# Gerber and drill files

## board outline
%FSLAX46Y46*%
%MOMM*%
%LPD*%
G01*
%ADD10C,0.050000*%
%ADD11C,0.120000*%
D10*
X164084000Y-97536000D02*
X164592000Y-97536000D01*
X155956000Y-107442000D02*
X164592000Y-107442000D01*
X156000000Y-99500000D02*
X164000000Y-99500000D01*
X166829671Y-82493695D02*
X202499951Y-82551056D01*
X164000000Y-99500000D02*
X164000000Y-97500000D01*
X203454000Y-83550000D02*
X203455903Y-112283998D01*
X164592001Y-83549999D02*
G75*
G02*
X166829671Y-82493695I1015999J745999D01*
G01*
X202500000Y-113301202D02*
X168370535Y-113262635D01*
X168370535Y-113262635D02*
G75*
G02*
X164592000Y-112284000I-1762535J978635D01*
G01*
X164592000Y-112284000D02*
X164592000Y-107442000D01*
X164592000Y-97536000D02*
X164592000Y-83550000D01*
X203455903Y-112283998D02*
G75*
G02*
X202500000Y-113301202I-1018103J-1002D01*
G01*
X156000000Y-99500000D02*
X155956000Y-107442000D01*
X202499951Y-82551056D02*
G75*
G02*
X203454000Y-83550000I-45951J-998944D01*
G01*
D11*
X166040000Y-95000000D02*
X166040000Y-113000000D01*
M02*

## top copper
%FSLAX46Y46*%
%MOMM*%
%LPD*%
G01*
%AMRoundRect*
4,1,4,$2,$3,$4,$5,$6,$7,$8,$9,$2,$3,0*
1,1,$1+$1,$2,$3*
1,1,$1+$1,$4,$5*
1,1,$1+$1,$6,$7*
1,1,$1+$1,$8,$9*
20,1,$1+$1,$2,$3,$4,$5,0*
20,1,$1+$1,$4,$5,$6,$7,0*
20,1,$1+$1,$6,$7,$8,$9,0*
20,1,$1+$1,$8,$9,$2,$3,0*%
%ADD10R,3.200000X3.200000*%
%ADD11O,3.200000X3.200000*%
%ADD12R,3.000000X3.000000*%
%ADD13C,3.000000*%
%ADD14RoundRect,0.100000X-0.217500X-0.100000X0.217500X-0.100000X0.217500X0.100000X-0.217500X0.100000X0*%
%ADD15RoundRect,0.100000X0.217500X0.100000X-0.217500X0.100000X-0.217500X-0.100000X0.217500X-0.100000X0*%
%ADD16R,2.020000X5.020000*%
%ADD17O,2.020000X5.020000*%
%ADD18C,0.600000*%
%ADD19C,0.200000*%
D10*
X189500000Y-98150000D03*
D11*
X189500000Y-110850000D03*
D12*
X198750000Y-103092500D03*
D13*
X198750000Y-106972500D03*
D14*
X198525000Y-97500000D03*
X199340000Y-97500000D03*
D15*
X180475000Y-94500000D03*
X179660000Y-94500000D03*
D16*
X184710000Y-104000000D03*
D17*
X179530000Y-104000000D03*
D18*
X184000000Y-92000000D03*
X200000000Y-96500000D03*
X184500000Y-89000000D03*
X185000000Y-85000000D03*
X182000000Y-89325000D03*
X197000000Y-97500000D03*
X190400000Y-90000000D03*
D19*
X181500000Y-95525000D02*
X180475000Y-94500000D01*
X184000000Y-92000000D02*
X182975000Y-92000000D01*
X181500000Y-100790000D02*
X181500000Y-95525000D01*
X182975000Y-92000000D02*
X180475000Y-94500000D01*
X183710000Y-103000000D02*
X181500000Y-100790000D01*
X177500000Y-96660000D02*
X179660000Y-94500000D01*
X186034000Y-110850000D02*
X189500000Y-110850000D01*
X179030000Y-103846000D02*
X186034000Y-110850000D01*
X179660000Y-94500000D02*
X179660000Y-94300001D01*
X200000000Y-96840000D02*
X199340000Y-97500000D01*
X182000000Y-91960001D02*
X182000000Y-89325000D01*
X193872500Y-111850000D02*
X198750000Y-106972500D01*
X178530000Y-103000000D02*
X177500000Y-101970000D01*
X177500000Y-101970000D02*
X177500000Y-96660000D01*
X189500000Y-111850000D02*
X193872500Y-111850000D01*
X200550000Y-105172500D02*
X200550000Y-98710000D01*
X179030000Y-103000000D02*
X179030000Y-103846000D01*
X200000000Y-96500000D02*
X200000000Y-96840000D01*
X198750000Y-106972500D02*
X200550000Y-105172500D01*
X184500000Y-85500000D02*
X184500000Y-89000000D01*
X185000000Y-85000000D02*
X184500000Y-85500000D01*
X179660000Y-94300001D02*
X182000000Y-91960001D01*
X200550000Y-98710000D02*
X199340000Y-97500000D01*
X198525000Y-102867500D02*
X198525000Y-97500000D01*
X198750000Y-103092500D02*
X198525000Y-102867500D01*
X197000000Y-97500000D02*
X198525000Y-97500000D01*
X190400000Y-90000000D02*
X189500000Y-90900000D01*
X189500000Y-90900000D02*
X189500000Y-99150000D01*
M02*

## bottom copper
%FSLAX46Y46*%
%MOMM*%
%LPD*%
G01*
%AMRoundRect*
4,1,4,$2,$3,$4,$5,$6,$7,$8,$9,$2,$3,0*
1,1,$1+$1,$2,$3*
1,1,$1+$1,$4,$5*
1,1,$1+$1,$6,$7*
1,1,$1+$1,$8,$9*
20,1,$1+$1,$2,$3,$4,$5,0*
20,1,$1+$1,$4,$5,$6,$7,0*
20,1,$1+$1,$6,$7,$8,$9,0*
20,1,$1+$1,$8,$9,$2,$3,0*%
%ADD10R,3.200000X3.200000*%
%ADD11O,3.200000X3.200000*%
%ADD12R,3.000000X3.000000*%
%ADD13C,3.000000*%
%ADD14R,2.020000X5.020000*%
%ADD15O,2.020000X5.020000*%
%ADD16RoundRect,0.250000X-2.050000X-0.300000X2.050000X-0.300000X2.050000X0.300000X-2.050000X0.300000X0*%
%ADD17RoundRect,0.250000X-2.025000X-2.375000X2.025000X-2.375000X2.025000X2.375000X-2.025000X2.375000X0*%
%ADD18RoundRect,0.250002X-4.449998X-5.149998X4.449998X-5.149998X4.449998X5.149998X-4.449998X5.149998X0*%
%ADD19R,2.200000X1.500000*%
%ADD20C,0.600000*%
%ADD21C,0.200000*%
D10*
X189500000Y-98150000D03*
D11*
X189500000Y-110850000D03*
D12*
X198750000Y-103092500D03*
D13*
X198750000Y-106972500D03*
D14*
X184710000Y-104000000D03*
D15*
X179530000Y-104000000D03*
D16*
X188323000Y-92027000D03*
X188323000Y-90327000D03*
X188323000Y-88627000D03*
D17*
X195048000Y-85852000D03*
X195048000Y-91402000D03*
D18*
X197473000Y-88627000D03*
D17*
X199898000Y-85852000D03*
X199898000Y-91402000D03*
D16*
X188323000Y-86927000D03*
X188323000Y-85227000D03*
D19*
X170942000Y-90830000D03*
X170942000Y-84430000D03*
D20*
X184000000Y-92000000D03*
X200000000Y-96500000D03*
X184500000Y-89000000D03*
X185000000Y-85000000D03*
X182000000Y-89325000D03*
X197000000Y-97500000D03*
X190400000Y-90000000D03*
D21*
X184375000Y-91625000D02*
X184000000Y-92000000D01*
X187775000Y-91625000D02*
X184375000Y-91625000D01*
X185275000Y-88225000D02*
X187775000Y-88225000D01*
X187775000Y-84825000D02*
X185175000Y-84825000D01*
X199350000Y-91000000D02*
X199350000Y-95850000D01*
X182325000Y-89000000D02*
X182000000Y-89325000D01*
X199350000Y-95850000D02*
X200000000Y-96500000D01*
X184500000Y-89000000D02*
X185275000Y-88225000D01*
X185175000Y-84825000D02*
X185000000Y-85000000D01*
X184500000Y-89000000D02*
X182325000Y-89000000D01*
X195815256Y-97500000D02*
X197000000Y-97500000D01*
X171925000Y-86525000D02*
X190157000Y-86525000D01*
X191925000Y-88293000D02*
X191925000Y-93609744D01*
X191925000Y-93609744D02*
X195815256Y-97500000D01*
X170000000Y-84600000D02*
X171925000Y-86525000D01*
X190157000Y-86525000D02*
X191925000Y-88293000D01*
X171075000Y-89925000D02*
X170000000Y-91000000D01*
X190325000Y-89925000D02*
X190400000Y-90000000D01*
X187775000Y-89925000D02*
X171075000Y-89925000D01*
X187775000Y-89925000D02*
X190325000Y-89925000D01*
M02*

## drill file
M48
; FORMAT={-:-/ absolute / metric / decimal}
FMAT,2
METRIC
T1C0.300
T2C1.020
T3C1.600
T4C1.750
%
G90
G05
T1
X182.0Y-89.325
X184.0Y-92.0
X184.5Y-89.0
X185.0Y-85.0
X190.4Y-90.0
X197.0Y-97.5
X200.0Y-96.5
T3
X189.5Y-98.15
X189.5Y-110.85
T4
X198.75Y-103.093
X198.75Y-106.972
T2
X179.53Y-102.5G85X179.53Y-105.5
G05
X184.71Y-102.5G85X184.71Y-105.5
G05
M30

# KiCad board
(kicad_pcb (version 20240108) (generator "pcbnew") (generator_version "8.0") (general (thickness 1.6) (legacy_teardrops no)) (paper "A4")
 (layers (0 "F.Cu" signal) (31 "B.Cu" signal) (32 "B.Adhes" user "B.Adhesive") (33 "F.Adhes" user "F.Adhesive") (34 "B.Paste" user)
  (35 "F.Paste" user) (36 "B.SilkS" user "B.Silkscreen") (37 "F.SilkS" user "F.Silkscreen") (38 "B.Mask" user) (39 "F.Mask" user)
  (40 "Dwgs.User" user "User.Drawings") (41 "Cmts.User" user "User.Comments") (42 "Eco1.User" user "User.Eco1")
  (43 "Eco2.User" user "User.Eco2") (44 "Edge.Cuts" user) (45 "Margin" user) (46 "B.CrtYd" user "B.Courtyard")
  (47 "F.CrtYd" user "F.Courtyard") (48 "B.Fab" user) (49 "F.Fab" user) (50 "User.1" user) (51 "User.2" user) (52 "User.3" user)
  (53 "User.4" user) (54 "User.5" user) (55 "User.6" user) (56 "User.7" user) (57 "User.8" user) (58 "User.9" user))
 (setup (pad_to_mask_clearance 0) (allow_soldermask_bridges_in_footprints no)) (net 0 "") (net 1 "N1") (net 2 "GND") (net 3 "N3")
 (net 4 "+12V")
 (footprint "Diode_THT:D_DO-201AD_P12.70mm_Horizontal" (layer "F.Cu") (at 189.5 98.15 -90)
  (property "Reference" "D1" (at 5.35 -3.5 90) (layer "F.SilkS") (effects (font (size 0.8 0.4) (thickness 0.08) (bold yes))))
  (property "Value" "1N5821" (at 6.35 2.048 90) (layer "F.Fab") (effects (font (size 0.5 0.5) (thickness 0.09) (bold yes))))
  (pad "1" thru_hole rect (at 0 0 270) (size 3.2 3.2) (drill 1.6) (layers "*.Cu" "*.Mask") (remove_unused_layers no) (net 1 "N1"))
  (pad "2" thru_hole oval (at 12.7 0 270) (size 3.2 3.2) (drill 1.6) (layers "*.Cu" "*.Mask") (remove_unused_layers no) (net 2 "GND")))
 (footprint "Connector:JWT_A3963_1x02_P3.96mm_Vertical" (layer "F.Cu") (at 198.75 103.0925 -90)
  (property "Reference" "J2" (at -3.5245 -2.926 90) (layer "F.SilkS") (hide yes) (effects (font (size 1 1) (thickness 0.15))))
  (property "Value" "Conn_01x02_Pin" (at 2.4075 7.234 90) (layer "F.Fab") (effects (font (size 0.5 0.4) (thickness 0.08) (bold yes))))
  (pad "1" thru_hole rect (at 0 0 270) (size 3 3) (drill 1.75) (layers "*.Cu" "*.Mask") (remove_unused_layers no) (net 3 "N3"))
  (pad "2" thru_hole circle (at 3.88 0 270) (size 3 3) (drill 1.75) (layers "*.Cu" "*.Mask") (remove_unused_layers no) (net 2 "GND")))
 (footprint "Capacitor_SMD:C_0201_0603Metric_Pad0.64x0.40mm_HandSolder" (layer "F.Cu") (at 198.9325 97.5)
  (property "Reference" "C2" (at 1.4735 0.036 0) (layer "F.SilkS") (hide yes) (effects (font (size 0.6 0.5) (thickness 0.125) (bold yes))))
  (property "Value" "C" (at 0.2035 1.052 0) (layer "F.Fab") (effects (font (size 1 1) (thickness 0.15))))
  (pad "" smd roundrect (at -0.4325 0) (size 0.458 0.36) (layers "F.Paste") (roundrect_rratio 0.25))
  (pad "" smd roundrect (at 0.4325 0) (size 0.458 0.36) (layers "F.Paste") (roundrect_rratio 0.25))
  (pad "1" smd roundrect (at -0.4075 0) (size 0.635 0.4) (layers "F.Cu" "F.Mask") (roundrect_rratio 0.25) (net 3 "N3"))
  (pad "2" smd roundrect (at 0.4075 0) (size 0.635 0.4) (layers "F.Cu" "F.Mask") (roundrect_rratio 0.25) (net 2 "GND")))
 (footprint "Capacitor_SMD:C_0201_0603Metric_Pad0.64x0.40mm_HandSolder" (layer "F.Cu") (at 180.0675 94.5 180)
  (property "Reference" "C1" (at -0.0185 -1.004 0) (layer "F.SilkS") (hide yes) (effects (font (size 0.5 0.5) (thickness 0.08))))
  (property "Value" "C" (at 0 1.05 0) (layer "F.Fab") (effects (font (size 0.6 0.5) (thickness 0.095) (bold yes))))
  (pad "" smd roundrect (at -0.4325 0 180) (size 0.458 0.36) (layers "F.Paste") (roundrect_rratio 0.25))
  (pad "" smd roundrect (at 0.4325 0 180) (size 0.458 0.36) (layers "F.Paste") (roundrect_rratio 0.25))
  (pad "1" smd roundrect (at -0.4075 0 180) (size 0.635 0.4) (layers "F.Cu" "F.Mask") (roundrect_rratio 0.25) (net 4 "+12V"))
  (pad "2" smd roundrect (at 0.4075 0 180) (size 0.635 0.4) (layers "F.Cu" "F.Mask") (roundrect_rratio 0.25) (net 2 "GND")))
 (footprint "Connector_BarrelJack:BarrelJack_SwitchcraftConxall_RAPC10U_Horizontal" (layer "F.Cu") (at 184.71 104)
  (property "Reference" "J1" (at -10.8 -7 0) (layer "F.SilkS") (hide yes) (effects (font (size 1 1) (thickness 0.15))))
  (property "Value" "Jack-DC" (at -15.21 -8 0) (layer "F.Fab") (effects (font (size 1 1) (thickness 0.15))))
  (fp_line (start -18.67 -9) (end -18.67 9) (stroke (width 0.12) (type solid)) (layer "Edge.Cuts"))
  (pad "1" thru_hole rect (at 0 0) (size 2.02 5.02) (drill oval 1.02 4.02) (layers "*.Cu" "*.Mask") (remove_unused_layers no) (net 4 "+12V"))
  (pad "2" thru_hole oval (at -5.18 0) (size 2.02 5.02) (drill oval 1.02 4.02) (layers "*.Cu" "*.Mask") (remove_unused_layers no)
   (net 2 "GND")))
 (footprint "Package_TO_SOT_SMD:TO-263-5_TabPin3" (layer "B.Cu") (at 195.973 88.627)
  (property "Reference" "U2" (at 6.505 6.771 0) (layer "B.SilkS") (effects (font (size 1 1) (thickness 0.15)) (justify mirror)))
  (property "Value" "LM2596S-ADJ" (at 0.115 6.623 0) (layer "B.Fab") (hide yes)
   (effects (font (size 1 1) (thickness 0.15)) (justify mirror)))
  (pad "1" smd roundrect (at -7.65 3.4) (size 4.6 1.1) (layers "B.Cu" "B.Paste" "B.Mask") (roundrect_rratio 0.227273) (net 4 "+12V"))
  (pad "2" smd roundrect (at -7.65 1.7) (size 4.6 1.1) (layers "B.Cu" "B.Paste" "B.Mask") (roundrect_rratio 0.227273) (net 1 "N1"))
  (pad "3" smd roundrect (at -7.65 0) (size 4.6 1.1) (layers "B.Cu" "B.Paste" "B.Mask") (roundrect_rratio 0.227273) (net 2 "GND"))
  (pad "3" smd roundrect (at -0.925 -2.775) (size 4.55 5.25) (layers "B.Cu" "B.Paste") (roundrect_rratio 0.054945) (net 2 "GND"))
  (pad "3" smd roundrect (at -0.925 2.775) (size 4.55 5.25) (layers "B.Cu" "B.Paste") (roundrect_rratio 0.054945) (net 2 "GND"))
  (pad "3" smd roundrect (at 1.5 0) (size 9.4 10.8) (layers "B.Cu" "B.Mask") (roundrect_rratio 0.026596) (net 2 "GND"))
  (pad "3" smd roundrect (at 3.925 -2.775) (size 4.55 5.25) (layers "B.Cu" "B.Paste") (roundrect_rratio 0.054945) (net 2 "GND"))
  (pad "3" smd roundrect (at 3.925 2.775) (size 4.55 5.25) (layers "B.Cu" "B.Paste") (roundrect_rratio 0.054945) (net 2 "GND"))
  (pad "4" smd roundrect (at -7.65 -1.7) (size 4.6 1.1) (layers "B.Cu" "B.Paste" "B.Mask") (roundrect_rratio 0.227273) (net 3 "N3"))
  (pad "5" smd roundrect (at -7.65 -3.4) (size 4.6 1.1) (layers "B.Cu" "B.Paste" "B.Mask") (roundrect_rratio 0.227273) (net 2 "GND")))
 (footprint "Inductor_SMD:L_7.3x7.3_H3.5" (layer "B.Cu") (at 170.942 87.63 90)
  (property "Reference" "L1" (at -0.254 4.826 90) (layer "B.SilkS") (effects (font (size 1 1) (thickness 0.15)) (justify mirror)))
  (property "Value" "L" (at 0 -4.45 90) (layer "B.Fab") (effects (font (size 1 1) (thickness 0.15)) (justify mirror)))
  (pad "1" smd rect (at -3.2 0 90) (size 1.5 2.2) (layers "B.Cu" "B.Paste" "B.Mask") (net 1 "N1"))
  (pad "2" smd rect (at 3.2 0 90) (size 1.5 2.2) (layers "B.Cu" "B.Paste" "B.Mask") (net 3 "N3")))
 (gr_line (start 164.084 97.536) (end 164.592 97.536) (stroke (width 0.05) (type default)) (layer "Edge.Cuts"))
 (gr_line (start 155.956 107.442) (end 164.592 107.442) (stroke (width 0.05) (type default)) (layer "Edge.Cuts"))
 (gr_line (start 156 99.5) (end 164 99.5) (stroke (width 0.05) (type default)) (layer "Edge.Cuts"))
 (gr_line (start 166.829671 82.493695) (end 202.499951 82.551056) (stroke (width 0.05) (type default)) (layer "Edge.Cuts"))
 (gr_line (start 164 99.5) (end 164 97.5) (stroke (width 0.05) (type default)) (layer "Edge.Cuts"))
 (gr_line (start 203.454 83.55) (end 203.455903 112.283998) (stroke (width 0.05) (type default)) (layer "Edge.Cuts"))
 (gr_arc (start 164.592001 83.549999) (mid 165.06993 81.664154) (end 166.829671 82.493695) (stroke (width 0.05) (type default))
  (layer "Edge.Cuts"))
 (gr_line (start 202.5 113.301202) (end 168.370535 113.262635) (stroke (width 0.05) (type default)) (layer "Edge.Cuts"))
 (gr_arc (start 168.370535 113.262635) (mid 166.102537 114.235605) (end 164.592 112.284) (stroke (width 0.05) (type default))
  (layer "Edge.Cuts"))
 (gr_line (start 164.592 112.284) (end 164.592 107.442) (stroke (width 0.05) (type default)) (layer "Edge.Cuts"))
 (gr_line (start 164.592 97.536) (end 164.592 83.55) (stroke (width 0.05) (type default)) (layer "Edge.Cuts"))
 (gr_arc (start 203.455903 112.283998) (mid 203.179716 112.982205) (end 202.5 113.301201) (stroke (width 0.05) (type default))
  (layer "Edge.Cuts"))
 (gr_line (start 156 99.5) (end 155.956 107.442) (stroke (width 0.05) (type default)) (layer "Edge.Cuts"))
 (gr_arc (start 202.499951 82.551056) (mid 203.177171 82.85933) (end 203.454 83.55) (stroke (width 0.05) (type default)) (layer "Edge.Cuts"))
 (segment (start 181.5 95.525) (end 180.475 94.5) (width 0.2) (layer "F.Cu") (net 4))
 (segment (start 184 92) (end 182.975 92) (width 0.2) (layer "F.Cu") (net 4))
 (segment (start 181.5 100.79) (end 181.5 95.525) (width 0.2) (layer "F.Cu") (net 4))
 (segment (start 182.975 92) (end 180.475 94.5) (width 0.2) (layer "F.Cu") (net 4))
 (segment (start 183.71 103) (end 181.5 100.79) (width 0.2) (layer "F.Cu") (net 4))
 (via (at 184 92) (size 0.6) (drill 0.3) (layers "F.Cu" "B.Cu") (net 4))
 (segment (start 184.375 91.625) (end 184 92) (width 0.2) (layer "B.Cu") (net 4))
 (segment (start 187.775 91.625) (end 184.375 91.625) (width 0.2) (layer "B.Cu") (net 4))
 (segment (start 177.5 96.66) (end 179.66 94.5) (width 0.2) (layer "F.Cu") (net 2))
 (segment (start 186.034 110.85) (end 189.5 110.85) (width 0.2) (layer "F.Cu") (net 2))
 (segment (start 179.03 103.846) (end 186.034 110.85) (width 0.2) (layer "F.Cu") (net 2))
 (segment (start 179.66 94.5) (end 179.66 94.300001) (width 0.2) (layer "F.Cu") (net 2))
 (segment (start 200 96.84) (end 199.34 97.5) (width 0.2) (layer "F.Cu") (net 2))
 (segment (start 182 91.960001) (end 182 89.325) (width 0.2) (layer "F.Cu") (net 2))
 (segment (start 193.8725 111.85) (end 198.75 106.9725) (width 0.2) (layer "F.Cu") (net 2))
 (segment (start 178.53 103) (end 177.5 101.97) (width 0.2) (layer "F.Cu") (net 2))
 (segment (start 177.5 101.97) (end 177.5 96.66) (width 0.2) (layer "F.Cu") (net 2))
 (segment (start 189.5 111.85) (end 193.8725 111.85) (width 0.2) (layer "F.Cu") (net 2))
 (segment (start 200.55 105.1725) (end 200.55 98.71) (width 0.2) (layer "F.Cu") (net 2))
 (segment (start 179.03 103) (end 179.03 103.846) (width 0.2) (layer "F.Cu") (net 2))
 (segment (start 200 96.5) (end 200 96.84) (width 0.2) (layer "F.Cu") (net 2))
 (segment (start 198.75 106.9725) (end 200.55 105.1725) (width 0.2) (layer "F.Cu") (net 2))
 (segment (start 184.5 85.5) (end 184.5 89) (width 0.2) (layer "F.Cu") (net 2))
 (segment (start 185 85) (end 184.5 85.5) (width 0.2) (layer "F.Cu") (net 2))
 (segment (start 179.66 94.300001) (end 182 91.960001) (width 0.2) (layer "F.Cu") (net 2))
 (segment (start 200.55 98.71) (end 199.34 97.5) (width 0.2) (layer "F.Cu") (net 2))
 (via (at 200 96.5) (size 0.6) (drill 0.3) (layers "F.Cu" "B.Cu") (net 2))
 (via (at 184.5 89) (size 0.6) (drill 0.3) (layers "F.Cu" "B.Cu") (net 2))
 (via (at 185 85) (size 0.6) (drill 0.3) (layers "F.Cu" "B.Cu") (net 2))
 (via (at 182 89.325) (size 0.6) (drill 0.3) (layers "F.Cu" "B.Cu") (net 2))
 (segment (start 185.275 88.225) (end 187.775 88.225) (width 0.2) (layer "B.Cu") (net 2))
 (segment (start 187.775 84.825) (end 185.175 84.825) (width 0.2) (layer "B.Cu") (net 2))
 (segment (start 199.35 91) (end 199.35 95.85) (width 0.2) (layer "B.Cu") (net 2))
 (segment (start 182.325 89) (end 182 89.325) (width 0.2) (layer "B.Cu") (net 2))
 (segment (start 199.35 95.85) (end 200 96.5) (width 0.2) (layer "B.Cu") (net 2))
 (segment (start 184.5 89) (end 185.275 88.225) (width 0.2) (layer "B.Cu") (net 2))
 (segment (start 185.175 84.825) (end 185 85) (width 0.2) (layer "B.Cu") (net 2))
 (segment (start 184.5 89) (end 182.325 89) (width 0.2) (layer "B.Cu") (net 2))
 (segment (start 198.525 102.8675) (end 198.525 97.5) (width 0.2) (layer "F.Cu") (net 3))
 (segment (start 198.75 103.0925) (end 198.525 102.8675) (width 0.2) (layer "F.Cu") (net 3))
 (segment (start 197 97.5) (end 198.525 97.5) (width 0.2) (layer "F.Cu") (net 3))
 (via (at 197 97.5) (size 0.6) (drill 0.3) (layers "F.Cu" "B.Cu") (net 3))
 (segment (start 195.815256 97.5) (end 197 97.5) (width 0.2) (layer "B.Cu") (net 3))
 (segment (start 171.925 86.525) (end 190.157 86.525) (width 0.2) (layer "B.Cu") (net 3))
 (segment (start 191.925 88.293) (end 191.925 93.609744) (width 0.2) (layer "B.Cu") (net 3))
 (segment (start 191.925 93.609744) (end 195.815256 97.5) (width 0.2) (layer "B.Cu") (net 3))
 (segment (start 170 84.6) (end 171.925 86.525) (width 0.2) (layer "B.Cu") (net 3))
 (segment (start 190.157 86.525) (end 191.925 88.293) (width 0.2) (layer "B.Cu") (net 3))
 (segment (start 190.4 90) (end 189.5 90.9) (width 0.2) (layer "F.Cu") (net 1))
 (segment (start 189.5 90.9) (end 189.5 99.15) (width 0.2) (layer "F.Cu") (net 1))
 (via (at 190.4 90) (size 0.6) (drill 0.3) (layers "F.Cu" "B.Cu") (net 1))
 (segment (start 171.075 89.925) (end 170 91) (width 0.2) (layer "B.Cu") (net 1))
 (segment (start 190.325 89.925) (end 190.4 90) (width 0.2) (layer "B.Cu") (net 1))
 (segment (start 187.775 89.925) (end 171.075 89.925) (width 0.2) (layer "B.Cu") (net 1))
 (segment (start 187.775 89.925) (end 190.325 89.925) (width 0.2) (layer "B.Cu") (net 1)))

